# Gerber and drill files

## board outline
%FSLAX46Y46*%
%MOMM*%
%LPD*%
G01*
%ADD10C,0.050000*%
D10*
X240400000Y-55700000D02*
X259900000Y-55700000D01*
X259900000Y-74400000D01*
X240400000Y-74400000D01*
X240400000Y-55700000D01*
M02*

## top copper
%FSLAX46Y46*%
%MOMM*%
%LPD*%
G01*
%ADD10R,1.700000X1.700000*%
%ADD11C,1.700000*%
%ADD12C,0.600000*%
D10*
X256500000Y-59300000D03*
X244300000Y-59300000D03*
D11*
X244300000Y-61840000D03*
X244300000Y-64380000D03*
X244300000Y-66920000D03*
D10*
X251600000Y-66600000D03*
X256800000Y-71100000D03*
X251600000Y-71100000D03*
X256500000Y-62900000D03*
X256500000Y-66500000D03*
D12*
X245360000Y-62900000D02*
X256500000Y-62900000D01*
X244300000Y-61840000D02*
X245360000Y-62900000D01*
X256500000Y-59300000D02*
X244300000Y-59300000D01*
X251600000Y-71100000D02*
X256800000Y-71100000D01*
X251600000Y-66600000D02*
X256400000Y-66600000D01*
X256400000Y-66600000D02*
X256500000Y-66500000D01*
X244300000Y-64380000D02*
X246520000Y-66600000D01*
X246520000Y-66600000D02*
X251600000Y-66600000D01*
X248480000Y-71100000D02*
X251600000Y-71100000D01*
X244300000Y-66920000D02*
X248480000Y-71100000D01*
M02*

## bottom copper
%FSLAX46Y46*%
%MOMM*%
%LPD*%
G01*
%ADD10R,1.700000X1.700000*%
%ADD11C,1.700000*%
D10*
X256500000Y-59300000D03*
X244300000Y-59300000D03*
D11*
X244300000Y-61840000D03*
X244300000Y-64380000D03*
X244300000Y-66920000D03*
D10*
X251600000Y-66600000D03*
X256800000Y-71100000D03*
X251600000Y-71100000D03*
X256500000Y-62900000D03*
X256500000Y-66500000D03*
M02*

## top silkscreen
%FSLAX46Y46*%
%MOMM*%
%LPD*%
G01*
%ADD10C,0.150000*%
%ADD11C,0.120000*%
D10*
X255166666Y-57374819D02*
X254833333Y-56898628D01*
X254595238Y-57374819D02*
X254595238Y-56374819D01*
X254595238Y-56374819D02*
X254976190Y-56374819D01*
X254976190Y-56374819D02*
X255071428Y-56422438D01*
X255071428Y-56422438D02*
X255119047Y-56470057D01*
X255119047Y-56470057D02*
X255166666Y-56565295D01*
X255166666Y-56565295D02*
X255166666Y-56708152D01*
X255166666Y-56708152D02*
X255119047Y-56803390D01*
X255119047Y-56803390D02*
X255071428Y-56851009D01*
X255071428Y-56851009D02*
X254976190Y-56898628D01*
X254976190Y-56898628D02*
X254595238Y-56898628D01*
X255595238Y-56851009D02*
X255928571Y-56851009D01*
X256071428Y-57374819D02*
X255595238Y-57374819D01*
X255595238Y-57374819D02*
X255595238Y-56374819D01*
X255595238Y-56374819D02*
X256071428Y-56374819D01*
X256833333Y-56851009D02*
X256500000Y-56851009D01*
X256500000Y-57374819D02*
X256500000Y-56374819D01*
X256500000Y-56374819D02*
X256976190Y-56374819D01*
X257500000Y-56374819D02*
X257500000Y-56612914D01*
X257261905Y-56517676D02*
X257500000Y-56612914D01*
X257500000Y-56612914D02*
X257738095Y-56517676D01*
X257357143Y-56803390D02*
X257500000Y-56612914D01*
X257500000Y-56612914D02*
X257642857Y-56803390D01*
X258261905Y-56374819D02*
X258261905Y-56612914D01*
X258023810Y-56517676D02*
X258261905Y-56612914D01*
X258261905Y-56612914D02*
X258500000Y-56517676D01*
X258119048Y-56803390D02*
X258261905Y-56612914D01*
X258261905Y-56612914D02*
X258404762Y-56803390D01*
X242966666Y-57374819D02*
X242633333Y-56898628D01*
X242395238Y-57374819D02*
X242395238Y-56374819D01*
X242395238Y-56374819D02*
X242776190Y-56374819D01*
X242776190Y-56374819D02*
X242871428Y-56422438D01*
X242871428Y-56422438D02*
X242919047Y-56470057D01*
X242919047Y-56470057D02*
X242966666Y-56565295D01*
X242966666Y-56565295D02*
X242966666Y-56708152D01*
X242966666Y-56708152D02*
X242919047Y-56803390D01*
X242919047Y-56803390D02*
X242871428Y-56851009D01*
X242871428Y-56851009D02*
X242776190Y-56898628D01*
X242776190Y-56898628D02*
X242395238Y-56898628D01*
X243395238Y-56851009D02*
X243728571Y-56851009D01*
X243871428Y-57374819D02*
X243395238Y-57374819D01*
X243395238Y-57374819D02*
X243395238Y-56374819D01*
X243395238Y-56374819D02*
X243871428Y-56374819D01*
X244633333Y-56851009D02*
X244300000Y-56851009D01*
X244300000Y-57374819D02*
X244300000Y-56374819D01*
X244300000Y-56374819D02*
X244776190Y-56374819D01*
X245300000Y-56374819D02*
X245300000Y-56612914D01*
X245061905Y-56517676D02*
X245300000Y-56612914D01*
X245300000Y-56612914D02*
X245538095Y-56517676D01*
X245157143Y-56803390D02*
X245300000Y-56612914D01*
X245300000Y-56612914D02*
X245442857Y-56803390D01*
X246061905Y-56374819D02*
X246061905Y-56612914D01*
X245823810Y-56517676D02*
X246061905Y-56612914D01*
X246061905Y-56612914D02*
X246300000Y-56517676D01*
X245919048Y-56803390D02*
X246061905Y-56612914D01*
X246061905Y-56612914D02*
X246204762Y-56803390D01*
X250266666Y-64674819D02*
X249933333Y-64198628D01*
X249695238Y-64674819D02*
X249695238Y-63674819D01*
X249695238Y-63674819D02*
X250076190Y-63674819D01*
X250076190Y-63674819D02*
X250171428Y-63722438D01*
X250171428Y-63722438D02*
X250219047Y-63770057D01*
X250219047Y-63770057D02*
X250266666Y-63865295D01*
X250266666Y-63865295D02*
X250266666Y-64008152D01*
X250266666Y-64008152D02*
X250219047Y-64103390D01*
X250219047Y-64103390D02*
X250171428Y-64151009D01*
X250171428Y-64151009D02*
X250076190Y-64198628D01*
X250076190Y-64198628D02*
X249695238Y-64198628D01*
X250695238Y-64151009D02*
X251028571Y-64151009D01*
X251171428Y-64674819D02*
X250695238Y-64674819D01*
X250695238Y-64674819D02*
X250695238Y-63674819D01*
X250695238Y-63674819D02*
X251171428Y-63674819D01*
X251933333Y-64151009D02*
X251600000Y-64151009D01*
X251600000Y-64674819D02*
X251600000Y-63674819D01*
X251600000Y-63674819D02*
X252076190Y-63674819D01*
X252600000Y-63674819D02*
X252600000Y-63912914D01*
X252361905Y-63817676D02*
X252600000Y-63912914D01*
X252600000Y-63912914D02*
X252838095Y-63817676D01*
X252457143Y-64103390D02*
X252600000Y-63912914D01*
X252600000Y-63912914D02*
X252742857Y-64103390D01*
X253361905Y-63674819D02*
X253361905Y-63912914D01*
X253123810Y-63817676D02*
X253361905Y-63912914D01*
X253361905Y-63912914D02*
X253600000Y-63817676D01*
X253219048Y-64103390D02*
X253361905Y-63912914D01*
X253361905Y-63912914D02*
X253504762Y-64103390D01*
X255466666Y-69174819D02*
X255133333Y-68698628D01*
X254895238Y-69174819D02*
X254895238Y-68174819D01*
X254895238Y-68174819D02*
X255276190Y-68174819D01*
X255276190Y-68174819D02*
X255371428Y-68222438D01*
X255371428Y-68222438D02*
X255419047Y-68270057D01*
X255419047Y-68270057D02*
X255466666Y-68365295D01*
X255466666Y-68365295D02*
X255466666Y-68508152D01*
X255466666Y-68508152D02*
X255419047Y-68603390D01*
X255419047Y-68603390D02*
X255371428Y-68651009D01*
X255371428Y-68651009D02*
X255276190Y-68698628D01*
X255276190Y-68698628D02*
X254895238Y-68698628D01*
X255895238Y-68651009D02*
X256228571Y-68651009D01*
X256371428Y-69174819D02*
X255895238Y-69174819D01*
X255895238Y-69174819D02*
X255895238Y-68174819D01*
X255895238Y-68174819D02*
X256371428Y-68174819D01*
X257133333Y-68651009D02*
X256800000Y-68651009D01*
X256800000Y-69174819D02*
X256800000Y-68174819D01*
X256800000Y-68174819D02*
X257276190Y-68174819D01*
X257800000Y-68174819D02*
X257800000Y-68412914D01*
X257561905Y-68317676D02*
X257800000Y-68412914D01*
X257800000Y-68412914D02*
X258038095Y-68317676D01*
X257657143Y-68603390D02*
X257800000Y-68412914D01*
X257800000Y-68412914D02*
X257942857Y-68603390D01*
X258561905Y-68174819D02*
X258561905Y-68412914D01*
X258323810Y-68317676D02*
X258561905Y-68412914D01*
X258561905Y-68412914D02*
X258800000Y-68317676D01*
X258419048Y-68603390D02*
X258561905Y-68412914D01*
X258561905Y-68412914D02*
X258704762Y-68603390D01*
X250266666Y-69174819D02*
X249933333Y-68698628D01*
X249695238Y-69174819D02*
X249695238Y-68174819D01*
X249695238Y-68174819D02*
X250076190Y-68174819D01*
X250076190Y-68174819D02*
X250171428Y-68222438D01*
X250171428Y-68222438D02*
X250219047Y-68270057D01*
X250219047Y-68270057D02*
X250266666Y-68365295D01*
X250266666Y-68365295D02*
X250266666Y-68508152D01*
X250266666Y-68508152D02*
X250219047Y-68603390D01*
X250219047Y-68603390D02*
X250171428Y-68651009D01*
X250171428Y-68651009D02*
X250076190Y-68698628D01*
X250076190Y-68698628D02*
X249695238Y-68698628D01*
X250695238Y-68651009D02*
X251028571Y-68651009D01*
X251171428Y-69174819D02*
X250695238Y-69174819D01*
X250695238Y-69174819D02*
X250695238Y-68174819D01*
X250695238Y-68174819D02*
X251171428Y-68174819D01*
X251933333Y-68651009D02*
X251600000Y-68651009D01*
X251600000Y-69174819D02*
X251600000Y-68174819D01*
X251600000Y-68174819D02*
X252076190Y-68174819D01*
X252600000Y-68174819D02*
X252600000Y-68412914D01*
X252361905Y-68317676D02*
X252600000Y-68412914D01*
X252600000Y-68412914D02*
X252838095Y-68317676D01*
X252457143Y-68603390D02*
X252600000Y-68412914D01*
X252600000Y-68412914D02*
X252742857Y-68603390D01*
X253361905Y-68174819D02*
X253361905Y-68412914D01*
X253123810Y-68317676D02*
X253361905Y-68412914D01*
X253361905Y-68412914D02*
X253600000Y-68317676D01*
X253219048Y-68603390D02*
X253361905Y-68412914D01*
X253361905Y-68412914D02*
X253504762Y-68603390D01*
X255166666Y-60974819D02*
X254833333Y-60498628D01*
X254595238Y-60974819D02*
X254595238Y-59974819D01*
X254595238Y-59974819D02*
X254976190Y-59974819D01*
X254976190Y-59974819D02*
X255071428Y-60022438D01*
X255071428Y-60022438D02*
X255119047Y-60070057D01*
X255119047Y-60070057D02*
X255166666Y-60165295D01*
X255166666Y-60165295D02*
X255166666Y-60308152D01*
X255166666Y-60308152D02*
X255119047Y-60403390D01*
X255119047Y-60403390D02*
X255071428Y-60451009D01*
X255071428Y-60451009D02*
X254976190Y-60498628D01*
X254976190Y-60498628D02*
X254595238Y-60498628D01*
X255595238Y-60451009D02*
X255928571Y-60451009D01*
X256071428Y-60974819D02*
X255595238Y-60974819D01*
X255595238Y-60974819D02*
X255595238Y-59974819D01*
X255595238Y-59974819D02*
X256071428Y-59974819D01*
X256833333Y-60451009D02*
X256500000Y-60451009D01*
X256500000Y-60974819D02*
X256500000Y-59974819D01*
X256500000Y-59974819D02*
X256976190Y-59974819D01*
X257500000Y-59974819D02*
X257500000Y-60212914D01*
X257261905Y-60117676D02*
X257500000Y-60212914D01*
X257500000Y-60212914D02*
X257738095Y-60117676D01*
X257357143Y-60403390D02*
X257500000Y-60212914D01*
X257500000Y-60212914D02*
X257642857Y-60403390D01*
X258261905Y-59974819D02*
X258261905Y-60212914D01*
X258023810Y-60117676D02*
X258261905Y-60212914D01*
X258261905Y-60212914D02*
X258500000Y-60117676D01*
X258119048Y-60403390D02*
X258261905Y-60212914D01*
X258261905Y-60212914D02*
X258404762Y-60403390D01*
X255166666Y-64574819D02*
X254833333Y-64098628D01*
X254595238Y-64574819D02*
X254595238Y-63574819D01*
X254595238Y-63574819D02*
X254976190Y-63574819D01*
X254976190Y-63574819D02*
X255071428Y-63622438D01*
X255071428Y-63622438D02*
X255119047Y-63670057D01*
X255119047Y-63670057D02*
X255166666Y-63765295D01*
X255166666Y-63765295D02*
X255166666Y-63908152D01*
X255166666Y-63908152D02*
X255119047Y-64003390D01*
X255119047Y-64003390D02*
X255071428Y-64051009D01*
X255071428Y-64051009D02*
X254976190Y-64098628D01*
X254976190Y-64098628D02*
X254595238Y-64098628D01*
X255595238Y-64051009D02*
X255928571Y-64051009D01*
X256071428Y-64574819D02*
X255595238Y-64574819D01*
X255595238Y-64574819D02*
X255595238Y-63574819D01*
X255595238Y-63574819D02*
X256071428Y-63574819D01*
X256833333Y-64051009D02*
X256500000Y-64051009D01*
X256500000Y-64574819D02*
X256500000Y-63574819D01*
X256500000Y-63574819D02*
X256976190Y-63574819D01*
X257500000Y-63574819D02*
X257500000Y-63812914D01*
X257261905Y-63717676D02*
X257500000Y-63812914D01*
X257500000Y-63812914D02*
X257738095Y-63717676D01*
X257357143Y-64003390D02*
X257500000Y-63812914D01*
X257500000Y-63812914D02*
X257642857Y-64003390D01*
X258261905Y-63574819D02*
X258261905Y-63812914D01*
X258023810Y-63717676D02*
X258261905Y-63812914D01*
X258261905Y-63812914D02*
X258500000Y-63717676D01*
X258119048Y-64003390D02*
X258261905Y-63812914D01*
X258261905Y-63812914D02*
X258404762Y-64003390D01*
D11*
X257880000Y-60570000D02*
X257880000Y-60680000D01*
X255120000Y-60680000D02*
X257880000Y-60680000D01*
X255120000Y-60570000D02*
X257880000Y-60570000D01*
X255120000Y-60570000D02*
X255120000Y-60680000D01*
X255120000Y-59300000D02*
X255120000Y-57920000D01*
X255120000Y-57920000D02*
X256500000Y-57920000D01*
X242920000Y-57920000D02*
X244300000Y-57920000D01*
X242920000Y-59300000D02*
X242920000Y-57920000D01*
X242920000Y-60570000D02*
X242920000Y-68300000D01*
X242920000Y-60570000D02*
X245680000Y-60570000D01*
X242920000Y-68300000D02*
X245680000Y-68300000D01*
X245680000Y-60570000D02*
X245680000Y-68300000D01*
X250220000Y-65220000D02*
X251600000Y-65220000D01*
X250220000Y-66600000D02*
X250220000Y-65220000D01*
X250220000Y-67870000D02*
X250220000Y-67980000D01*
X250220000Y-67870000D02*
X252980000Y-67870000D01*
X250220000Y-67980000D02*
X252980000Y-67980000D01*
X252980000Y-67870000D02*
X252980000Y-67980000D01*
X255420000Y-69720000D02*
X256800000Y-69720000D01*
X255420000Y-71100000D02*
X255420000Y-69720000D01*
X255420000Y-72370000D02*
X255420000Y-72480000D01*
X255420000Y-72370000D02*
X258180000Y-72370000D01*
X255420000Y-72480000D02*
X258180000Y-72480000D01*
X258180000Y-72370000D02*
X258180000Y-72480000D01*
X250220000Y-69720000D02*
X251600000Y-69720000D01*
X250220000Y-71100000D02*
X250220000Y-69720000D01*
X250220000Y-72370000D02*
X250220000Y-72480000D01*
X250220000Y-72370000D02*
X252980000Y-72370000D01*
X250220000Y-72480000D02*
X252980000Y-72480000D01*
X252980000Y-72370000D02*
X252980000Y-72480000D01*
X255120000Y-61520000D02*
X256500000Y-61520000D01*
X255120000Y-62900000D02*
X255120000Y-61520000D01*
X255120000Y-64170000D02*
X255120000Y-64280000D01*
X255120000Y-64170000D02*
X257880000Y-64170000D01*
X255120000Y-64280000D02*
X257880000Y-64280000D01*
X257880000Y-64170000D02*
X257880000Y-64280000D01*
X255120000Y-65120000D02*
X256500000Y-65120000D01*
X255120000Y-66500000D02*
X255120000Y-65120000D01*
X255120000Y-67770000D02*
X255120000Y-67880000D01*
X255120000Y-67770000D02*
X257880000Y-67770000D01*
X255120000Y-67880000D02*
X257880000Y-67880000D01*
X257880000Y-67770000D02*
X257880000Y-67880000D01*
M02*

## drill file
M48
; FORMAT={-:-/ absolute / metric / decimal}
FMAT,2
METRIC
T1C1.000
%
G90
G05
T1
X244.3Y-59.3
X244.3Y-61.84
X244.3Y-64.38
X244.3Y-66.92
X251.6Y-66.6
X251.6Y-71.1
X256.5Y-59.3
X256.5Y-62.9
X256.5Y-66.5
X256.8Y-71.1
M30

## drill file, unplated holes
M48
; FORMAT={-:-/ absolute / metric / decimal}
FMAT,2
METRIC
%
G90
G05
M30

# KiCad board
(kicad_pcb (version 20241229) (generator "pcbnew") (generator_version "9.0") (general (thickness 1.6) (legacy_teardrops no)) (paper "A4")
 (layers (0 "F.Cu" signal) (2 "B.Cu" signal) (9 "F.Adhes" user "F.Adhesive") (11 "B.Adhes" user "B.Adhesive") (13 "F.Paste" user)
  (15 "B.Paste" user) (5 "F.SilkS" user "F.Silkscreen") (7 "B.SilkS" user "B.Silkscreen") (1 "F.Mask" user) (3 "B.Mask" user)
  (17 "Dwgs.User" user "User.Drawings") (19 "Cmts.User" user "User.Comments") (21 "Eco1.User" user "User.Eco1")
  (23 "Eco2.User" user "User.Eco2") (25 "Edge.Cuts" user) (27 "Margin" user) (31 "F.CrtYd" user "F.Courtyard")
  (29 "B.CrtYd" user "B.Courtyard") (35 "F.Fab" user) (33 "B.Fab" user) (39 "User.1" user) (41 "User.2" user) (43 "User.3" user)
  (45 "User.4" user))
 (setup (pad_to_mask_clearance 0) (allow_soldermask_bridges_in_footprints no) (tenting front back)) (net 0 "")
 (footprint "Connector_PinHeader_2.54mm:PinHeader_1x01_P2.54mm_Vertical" (layer "F.Cu") (at 256.5 62.9)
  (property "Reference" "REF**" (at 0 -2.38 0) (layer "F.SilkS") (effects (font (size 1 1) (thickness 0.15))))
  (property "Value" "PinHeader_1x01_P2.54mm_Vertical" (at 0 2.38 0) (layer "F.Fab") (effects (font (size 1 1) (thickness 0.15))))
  (fp_line (start -1.38 -1.38) (end 0 -1.38) (stroke (width 0.12) (type solid)) (layer "F.SilkS") (net 1))
  (fp_line (start -1.38 0) (end -1.38 -1.38) (stroke (width 0.12) (type solid)) (layer "F.SilkS") (net 1))
  (fp_line (start -1.38 1.27) (end -1.38 1.38) (stroke (width 0.12) (type solid)) (layer "F.SilkS") (net 1))
  (fp_line (start -1.38 1.27) (end 1.38 1.27) (stroke (width 0.12) (type solid)) (layer "F.SilkS") (net 1))
  (fp_line (start -1.38 1.38) (end 1.38 1.38) (stroke (width 0.12) (type solid)) (layer "F.SilkS") (net 1))
  (fp_line (start 1.38 1.27) (end 1.38 1.38) (stroke (width 0.12) (type solid)) (layer "F.SilkS") (net 1))
  (pad "1" thru_hole rect (at 0 0) (size 1.7 1.7) (drill 1) (layers "*.Cu" "*.Mask") (remove_unused_layers no)))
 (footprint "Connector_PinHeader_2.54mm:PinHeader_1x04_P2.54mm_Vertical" (layer "F.Cu") (at 244.3 59.3)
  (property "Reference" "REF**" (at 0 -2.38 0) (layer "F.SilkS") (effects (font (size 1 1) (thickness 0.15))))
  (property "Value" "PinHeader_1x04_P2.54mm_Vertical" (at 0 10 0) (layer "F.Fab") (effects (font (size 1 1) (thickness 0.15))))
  (fp_line (start -1.38 -1.38) (end 0 -1.38) (stroke (width 0.12) (type solid)) (layer "F.SilkS") (net 1))
  (fp_line (start -1.38 0) (end -1.38 -1.38) (stroke (width 0.12) (type solid)) (layer "F.SilkS") (net 1))
  (fp_line (start -1.38 1.27) (end -1.38 9) (stroke (width 0.12) (type solid)) (layer "F.SilkS") (net 1))
  (fp_line (start -1.38 1.27) (end 1.38 1.27) (stroke (width 0.12) (type solid)) (layer "F.SilkS") (net 1))
  (fp_line (start -1.38 9) (end 1.38 9) (stroke (width 0.12) (type solid)) (layer "F.SilkS") (net 1))
  (fp_line (start 1.38 1.27) (end 1.38 9) (stroke (width 0.12) (type solid)) (layer "F.SilkS") (net 1))
  (pad "1" thru_hole rect (at 0 0) (size 1.7 1.7) (drill 1) (layers "*.Cu" "*.Mask") (remove_unused_layers no))
  (pad "2" thru_hole circle (at 0 2.54) (size 1.7 1.7) (drill 1) (layers "*.Cu" "*.Mask") (remove_unused_layers no))
  (pad "3" thru_hole circle (at 0 5.08) (size 1.7 1.7) (drill 1) (layers "*.Cu" "*.Mask") (remove_unused_layers no))
  (pad "4" thru_hole circle (at 0 7.62) (size 1.7 1.7) (drill 1) (layers "*.Cu" "*.Mask") (remove_unused_layers no)))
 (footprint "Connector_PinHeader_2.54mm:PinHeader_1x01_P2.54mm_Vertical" (layer "F.Cu") (at 256.5 66.5)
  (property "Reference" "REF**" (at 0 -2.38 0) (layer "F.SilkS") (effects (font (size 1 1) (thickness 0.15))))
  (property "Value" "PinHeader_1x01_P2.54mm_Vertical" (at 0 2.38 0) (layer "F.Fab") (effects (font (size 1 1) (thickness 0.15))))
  (fp_line (start -1.38 -1.38) (end 0 -1.38) (stroke (width 0.12) (type solid)) (layer "F.SilkS") (net 1))
  (fp_line (start -1.38 0) (end -1.38 -1.38) (stroke (width 0.12) (type solid)) (layer "F.SilkS") (net 1))
  (fp_line (start -1.38 1.27) (end -1.38 1.38) (stroke (width 0.12) (type solid)) (layer "F.SilkS") (net 1))
  (fp_line (start -1.38 1.27) (end 1.38 1.27) (stroke (width 0.12) (type solid)) (layer "F.SilkS") (net 1))
  (fp_line (start -1.38 1.38) (end 1.38 1.38) (stroke (width 0.12) (type solid)) (layer "F.SilkS") (net 1))
  (fp_line (start 1.38 1.27) (end 1.38 1.38) (stroke (width 0.12) (type solid)) (layer "F.SilkS") (net 1))
  (pad "1" thru_hole rect (at 0 0) (size 1.7 1.7) (drill 1) (layers "*.Cu" "*.Mask") (remove_unused_layers no)))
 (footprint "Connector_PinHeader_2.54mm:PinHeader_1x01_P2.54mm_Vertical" (layer "F.Cu") (at 256.5 59.3)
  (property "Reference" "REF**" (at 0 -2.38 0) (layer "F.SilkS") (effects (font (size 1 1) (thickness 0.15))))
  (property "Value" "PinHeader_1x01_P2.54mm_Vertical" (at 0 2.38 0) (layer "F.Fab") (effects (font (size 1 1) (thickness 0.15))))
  (fp_line (start -1.38 -1.38) (end 0 -1.38) (stroke (width 0.12) (type solid)) (layer "F.SilkS") (net 1))
  (fp_line (start -1.38 0) (end -1.38 -1.38) (stroke (width 0.12) (type solid)) (layer "F.SilkS") (net 1))
  (fp_line (start -1.38 1.27) (end -1.38 1.38) (stroke (width 0.12) (type solid)) (layer "F.SilkS") (net 1))
  (fp_line (start -1.38 1.27) (end 1.38 1.27) (stroke (width 0.12) (type solid)) (layer "F.SilkS") (net 1))
  (fp_line (start -1.38 1.38) (end 1.38 1.38) (stroke (width 0.12) (type solid)) (layer "F.SilkS") (net 1))
  (fp_line (start 1.38 1.27) (end 1.38 1.38) (stroke (width 0.12) (type solid)) (layer "F.SilkS") (net 1))
  (pad "1" thru_hole rect (at 0 0) (size 1.7 1.7) (drill 1) (layers "*.Cu" "*.Mask") (remove_unused_layers no)))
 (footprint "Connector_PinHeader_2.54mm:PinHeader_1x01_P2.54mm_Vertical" (layer "F.Cu") (at 251.6 71.1)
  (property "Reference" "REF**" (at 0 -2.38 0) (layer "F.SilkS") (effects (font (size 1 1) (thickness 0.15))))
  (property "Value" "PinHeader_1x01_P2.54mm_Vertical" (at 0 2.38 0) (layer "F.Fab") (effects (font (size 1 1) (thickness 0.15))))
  (fp_line (start -1.38 -1.38) (end 0 -1.38) (stroke (width 0.12) (type solid)) (layer "F.SilkS") (net 1))
  (fp_line (start -1.38 0) (end -1.38 -1.38) (stroke (width 0.12) (type solid)) (layer "F.SilkS") (net 1))
  (fp_line (start -1.38 1.27) (end -1.38 1.38) (stroke (width 0.12) (type solid)) (layer "F.SilkS") (net 1))
  (fp_line (start -1.38 1.27) (end 1.38 1.27) (stroke (width 0.12) (type solid)) (layer "F.SilkS") (net 1))
  (fp_line (start -1.38 1.38) (end 1.38 1.38) (stroke (width 0.12) (type solid)) (layer "F.SilkS") (net 1))
  (fp_line (start 1.38 1.27) (end 1.38 1.38) (stroke (width 0.12) (type solid)) (layer "F.SilkS") (net 1))
  (pad "1" thru_hole rect (at 0 0) (size 1.7 1.7) (drill 1) (layers "*.Cu" "*.Mask") (remove_unused_layers no)))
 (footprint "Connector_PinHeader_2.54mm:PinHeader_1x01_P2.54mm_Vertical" (layer "F.Cu") (at 251.6 66.6)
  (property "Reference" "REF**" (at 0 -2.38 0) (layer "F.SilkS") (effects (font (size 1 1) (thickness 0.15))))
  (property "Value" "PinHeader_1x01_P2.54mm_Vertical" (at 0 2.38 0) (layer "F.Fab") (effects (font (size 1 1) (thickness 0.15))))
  (fp_line (start -1.38 -1.38) (end 0 -1.38) (stroke (width 0.12) (type solid)) (layer "F.SilkS") (net 1))
  (fp_line (start -1.38 0) (end -1.38 -1.38) (stroke (width 0.12) (type solid)) (layer "F.SilkS") (net 1))
  (fp_line (start -1.38 1.27) (end -1.38 1.38) (stroke (width 0.12) (type solid)) (layer "F.SilkS") (net 1))
  (fp_line (start -1.38 1.27) (end 1.38 1.27) (stroke (width 0.12) (type solid)) (layer "F.SilkS") (net 1))
  (fp_line (start -1.38 1.38) (end 1.38 1.38) (stroke (width 0.12) (type solid)) (layer "F.SilkS") (net 1))
  (fp_line (start 1.38 1.27) (end 1.38 1.38) (stroke (width 0.12) (type solid)) (layer "F.SilkS") (net 1))
  (pad "1" thru_hole rect (at 0 0) (size 1.7 1.7) (drill 1) (layers "*.Cu" "*.Mask") (remove_unused_layers no)))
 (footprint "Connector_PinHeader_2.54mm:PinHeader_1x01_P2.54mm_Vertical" (layer "F.Cu") (at 256.8 71.1)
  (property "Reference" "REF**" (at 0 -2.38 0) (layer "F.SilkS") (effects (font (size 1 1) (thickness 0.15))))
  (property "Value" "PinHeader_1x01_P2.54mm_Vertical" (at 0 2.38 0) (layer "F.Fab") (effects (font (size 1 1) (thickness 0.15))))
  (fp_line (start -1.38 -1.38) (end 0 -1.38) (stroke (width 0.12) (type solid)) (layer "F.SilkS") (net 1))
  (fp_line (start -1.38 0) (end -1.38 -1.38) (stroke (width 0.12) (type solid)) (layer "F.SilkS") (net 1))
  (fp_line (start -1.38 1.27) (end -1.38 1.38) (stroke (width 0.12) (type solid)) (layer "F.SilkS") (net 1))
  (fp_line (start -1.38 1.27) (end 1.38 1.27) (stroke (width 0.12) (type solid)) (layer "F.SilkS") (net 1))
  (fp_line (start -1.38 1.38) (end 1.38 1.38) (stroke (width 0.12) (type solid)) (layer "F.SilkS") (net 1))
  (fp_line (start 1.38 1.27) (end 1.38 1.38) (stroke (width 0.12) (type solid)) (layer "F.SilkS") (net 1))
  (pad "1" thru_hole rect (at 0 0) (size 1.7 1.7) (drill 1) (layers "*.Cu" "*.Mask") (remove_unused_layers no)))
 (gr_rect (start 240.4 55.7) (end 259.9 74.4) (stroke (width 0.05) (type default)) (fill no) (layer "Edge.Cuts"))
 (segment (start 251.6 71.1) (end 256.8 71.1) (width 0.6) (layer "F.Cu") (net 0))
 (segment (start 256.4 66.6) (end 256.5 66.5) (width 0.6) (layer "F.Cu") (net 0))
 (segment (start 244.3 64.38) (end 246.52 66.6) (width 0.6) (layer "F.Cu") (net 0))
 (segment (start 246.52 66.6) (end 251.6 66.6) (width 0.6) (layer "F.Cu") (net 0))
 (segment (start 248.48 71.1) (end 251.6 71.1) (width 0.6) (layer "F.Cu") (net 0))
 (segment (start 244.3 61.84) (end 245.36 62.9) (width 0.6) (layer "F.Cu") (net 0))
 (segment (start 244.3 66.92) (end 248.48 71.1) (width 0.6) (layer "F.Cu") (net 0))
 (segment (start 251.6 66.6) (end 256.4 66.6) (width 0.6) (layer "F.Cu") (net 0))
 (segment (start 245.36 62.9) (end 256.5 62.9) (width 0.6) (layer "F.Cu") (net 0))
 (segment (start 256.5 59.3) (end 244.3 59.3) (width 0.6) (layer "F.Cu") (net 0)))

